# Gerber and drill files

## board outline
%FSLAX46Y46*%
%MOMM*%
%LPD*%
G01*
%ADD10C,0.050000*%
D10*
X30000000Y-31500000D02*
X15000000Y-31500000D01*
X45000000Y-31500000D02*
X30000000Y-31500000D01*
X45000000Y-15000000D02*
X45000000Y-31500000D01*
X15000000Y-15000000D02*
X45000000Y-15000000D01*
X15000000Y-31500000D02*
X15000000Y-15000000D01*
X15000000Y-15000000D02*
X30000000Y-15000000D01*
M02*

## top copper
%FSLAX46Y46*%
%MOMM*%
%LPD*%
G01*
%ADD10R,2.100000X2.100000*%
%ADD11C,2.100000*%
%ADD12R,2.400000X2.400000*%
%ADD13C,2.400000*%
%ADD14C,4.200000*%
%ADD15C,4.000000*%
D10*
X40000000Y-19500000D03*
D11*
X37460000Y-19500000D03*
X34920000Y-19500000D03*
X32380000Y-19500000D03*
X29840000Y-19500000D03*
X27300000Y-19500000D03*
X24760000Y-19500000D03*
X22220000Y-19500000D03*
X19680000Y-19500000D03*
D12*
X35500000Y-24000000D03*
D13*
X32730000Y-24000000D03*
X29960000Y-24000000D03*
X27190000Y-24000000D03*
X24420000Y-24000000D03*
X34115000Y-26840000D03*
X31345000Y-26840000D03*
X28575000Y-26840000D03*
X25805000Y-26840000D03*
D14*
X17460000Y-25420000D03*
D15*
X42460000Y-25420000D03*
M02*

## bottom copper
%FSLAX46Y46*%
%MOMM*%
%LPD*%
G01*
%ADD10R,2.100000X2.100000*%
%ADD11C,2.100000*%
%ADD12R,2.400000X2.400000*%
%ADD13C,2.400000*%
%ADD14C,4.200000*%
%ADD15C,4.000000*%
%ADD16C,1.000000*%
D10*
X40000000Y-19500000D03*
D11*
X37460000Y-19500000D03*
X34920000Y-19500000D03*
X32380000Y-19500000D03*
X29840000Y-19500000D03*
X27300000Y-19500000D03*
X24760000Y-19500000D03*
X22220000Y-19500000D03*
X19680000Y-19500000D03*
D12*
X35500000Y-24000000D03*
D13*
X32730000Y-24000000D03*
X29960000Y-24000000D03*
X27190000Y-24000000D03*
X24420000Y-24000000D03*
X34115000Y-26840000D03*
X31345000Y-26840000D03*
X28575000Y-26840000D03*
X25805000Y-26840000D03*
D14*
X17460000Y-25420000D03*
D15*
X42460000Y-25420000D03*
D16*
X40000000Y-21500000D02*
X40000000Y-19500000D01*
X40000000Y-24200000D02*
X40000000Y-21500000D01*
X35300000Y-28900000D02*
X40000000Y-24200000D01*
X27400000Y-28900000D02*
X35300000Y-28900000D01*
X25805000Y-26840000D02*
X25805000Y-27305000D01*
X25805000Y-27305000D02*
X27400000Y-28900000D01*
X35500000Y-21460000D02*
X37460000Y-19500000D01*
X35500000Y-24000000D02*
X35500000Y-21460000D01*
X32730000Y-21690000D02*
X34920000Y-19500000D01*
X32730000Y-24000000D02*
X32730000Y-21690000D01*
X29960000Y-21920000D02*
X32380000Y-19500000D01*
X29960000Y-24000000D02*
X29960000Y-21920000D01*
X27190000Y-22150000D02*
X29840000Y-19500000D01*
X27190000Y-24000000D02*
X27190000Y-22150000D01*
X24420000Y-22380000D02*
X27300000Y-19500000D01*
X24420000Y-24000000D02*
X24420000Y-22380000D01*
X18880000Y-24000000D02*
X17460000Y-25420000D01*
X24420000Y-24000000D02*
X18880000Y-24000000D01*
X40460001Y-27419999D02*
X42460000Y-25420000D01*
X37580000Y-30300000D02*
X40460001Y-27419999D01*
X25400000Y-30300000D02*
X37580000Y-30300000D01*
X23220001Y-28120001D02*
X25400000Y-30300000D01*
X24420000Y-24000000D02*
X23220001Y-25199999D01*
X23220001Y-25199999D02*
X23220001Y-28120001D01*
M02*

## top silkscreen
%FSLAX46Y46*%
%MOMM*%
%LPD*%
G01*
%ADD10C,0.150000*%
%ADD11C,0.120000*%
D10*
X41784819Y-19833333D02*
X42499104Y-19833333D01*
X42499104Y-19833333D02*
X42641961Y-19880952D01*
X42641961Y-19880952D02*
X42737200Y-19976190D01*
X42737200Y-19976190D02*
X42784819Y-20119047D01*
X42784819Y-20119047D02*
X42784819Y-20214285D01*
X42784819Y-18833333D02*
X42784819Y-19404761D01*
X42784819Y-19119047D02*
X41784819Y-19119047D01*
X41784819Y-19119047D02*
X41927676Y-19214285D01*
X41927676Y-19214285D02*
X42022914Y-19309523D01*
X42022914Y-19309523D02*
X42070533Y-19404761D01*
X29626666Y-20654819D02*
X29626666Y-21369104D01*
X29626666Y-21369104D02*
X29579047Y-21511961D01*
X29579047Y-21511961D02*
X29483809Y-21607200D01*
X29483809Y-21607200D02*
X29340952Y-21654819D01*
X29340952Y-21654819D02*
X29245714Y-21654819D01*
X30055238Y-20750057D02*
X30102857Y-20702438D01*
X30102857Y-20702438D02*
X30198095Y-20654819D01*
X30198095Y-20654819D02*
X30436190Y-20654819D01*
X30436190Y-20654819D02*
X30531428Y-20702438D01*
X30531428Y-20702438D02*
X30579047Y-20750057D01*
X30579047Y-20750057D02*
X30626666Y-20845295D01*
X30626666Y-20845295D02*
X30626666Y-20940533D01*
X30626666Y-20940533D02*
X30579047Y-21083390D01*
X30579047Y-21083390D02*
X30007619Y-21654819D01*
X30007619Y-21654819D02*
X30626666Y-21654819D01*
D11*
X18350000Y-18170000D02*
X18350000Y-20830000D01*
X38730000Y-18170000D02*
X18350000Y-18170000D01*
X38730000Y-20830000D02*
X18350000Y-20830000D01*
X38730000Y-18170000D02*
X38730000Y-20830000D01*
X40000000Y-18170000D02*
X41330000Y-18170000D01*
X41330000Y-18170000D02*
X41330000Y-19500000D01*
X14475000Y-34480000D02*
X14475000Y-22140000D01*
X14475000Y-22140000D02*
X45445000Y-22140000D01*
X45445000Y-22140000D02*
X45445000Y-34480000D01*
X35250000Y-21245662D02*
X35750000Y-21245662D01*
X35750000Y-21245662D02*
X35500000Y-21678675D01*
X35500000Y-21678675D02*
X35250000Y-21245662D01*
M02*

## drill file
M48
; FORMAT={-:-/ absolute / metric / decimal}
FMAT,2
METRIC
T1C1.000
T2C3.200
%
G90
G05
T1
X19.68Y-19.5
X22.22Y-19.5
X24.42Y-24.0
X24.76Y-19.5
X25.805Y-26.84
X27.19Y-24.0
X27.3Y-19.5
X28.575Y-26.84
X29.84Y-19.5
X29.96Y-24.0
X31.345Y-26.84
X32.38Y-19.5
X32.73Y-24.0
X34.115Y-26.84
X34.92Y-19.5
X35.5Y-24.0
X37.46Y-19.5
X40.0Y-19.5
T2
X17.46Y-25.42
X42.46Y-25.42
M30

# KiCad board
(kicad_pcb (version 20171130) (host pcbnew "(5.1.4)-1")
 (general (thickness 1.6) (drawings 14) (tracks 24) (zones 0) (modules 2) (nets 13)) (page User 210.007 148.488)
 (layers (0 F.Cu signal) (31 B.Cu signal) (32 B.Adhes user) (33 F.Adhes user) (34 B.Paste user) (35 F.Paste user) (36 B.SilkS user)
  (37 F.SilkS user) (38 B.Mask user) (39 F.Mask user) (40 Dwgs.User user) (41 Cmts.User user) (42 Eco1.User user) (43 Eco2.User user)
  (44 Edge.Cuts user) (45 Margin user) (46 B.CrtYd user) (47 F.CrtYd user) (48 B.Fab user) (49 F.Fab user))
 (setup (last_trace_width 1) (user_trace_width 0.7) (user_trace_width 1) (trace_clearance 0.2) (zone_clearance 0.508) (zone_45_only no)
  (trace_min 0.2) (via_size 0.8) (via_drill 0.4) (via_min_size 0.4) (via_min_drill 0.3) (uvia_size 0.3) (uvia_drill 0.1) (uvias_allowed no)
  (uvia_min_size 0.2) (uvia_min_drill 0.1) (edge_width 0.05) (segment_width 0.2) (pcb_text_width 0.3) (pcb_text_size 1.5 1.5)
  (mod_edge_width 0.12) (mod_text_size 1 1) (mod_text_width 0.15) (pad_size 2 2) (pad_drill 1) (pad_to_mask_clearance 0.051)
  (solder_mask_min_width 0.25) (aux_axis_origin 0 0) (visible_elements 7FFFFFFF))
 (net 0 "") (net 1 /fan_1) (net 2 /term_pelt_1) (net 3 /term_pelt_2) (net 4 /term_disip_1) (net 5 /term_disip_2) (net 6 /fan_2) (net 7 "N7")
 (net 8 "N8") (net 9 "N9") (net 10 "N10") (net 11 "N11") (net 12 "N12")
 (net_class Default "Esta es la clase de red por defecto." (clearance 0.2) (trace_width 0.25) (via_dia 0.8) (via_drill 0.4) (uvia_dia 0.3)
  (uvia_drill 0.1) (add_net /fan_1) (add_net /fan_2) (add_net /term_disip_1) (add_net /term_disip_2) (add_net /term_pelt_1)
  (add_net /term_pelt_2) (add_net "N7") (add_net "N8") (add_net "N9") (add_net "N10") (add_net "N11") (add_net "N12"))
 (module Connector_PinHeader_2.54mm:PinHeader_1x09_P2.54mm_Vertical (layer F.Cu) (at 40 19.5 270)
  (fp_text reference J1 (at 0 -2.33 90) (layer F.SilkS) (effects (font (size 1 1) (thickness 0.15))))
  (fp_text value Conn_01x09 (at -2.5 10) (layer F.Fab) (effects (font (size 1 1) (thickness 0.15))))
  (fp_line (start -1.33 21.65) (end 1.33 21.65) (layer F.SilkS) (width 0.12))
  (fp_line (start -1.33 1.27) (end -1.33 21.65) (layer F.SilkS) (width 0.12))
  (fp_line (start 1.33 1.27) (end 1.33 21.65) (layer F.SilkS) (width 0.12))
  (fp_line (start -1.33 1.27) (end 1.33 1.27) (layer F.SilkS) (width 0.12))
  (fp_line (start -1.33 0) (end -1.33 -1.33) (layer F.SilkS) (width 0.12))
  (fp_line (start -1.33 -1.33) (end 0 -1.33) (layer F.SilkS) (width 0.12))
  (pad 1 thru_hole rect (at 0 0 270) (size 2.1 2.1) (drill 1) (layers *.Cu *.Mask) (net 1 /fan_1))
  (pad 2 thru_hole circle (at 0 2.54 270) (size 2.1 2.1) (drill 1) (layers *.Cu *.Mask) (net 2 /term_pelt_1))
  (pad 3 thru_hole circle (at 0 5.08 270) (size 2.1 2.1) (drill 1) (layers *.Cu *.Mask) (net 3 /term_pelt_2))
  (pad 4 thru_hole circle (at 0 7.62 270) (size 2.1 2.1) (drill 1) (layers *.Cu *.Mask) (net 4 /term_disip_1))
  (pad 5 thru_hole circle (at 0 10.16 270) (size 2.1 2.1) (drill 1) (layers *.Cu *.Mask) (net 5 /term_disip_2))
  (pad 6 thru_hole circle (at 0 12.7 270) (size 2.1 2.1) (drill 1) (layers *.Cu *.Mask) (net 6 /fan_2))
  (pad 7 thru_hole circle (at 0 15.24 270) (size 2.1 2.1) (drill 1) (layers *.Cu *.Mask) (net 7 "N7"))
  (pad 8 thru_hole circle (at 0 17.78 270) (size 2.1 2.1) (drill 1) (layers *.Cu *.Mask) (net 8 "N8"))
  (pad 9 thru_hole circle (at 0 20.32 270) (size 2.1 2.1) (drill 1) (layers *.Cu *.Mask) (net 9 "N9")))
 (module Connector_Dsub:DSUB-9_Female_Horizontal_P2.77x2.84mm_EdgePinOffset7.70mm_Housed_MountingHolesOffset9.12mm (layer F.Cu) (at 35.5 24)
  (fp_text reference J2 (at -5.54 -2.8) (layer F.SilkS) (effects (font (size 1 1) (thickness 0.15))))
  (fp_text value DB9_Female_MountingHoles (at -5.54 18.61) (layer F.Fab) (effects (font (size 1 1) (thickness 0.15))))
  (fp_line (start -21.025 10.48) (end -21.025 -1.86) (layer F.SilkS) (width 0.12))
  (fp_line (start -21.025 -1.86) (end 9.945 -1.86) (layer F.SilkS) (width 0.12))
  (fp_line (start 9.945 -1.86) (end 9.945 10.48) (layer F.SilkS) (width 0.12))
  (fp_line (start -0.25 -2.754338) (end 0.25 -2.754338) (layer F.SilkS) (width 0.12))
  (fp_line (start 0.25 -2.754338) (end 0 -2.321325) (layer F.SilkS) (width 0.12))
  (fp_line (start 0 -2.321325) (end -0.25 -2.754338) (layer F.SilkS) (width 0.12))
  (pad 1 thru_hole rect (at 0 0) (size 2.4 2.4) (drill 1) (layers *.Cu *.Mask) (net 2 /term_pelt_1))
  (pad 2 thru_hole circle (at -2.77 0) (size 2.4 2.4) (drill 1) (layers *.Cu *.Mask) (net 3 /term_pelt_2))
  (pad 3 thru_hole circle (at -5.54 0) (size 2.4 2.4) (drill 1) (layers *.Cu *.Mask) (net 4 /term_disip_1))
  (pad 4 thru_hole circle (at -8.31 0) (size 2.4 2.4) (drill 1) (layers *.Cu *.Mask) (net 5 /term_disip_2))
  (pad 5 thru_hole circle (at -11.08 0) (size 2.4 2.4) (drill 1) (layers *.Cu *.Mask) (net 6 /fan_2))
  (pad 6 thru_hole circle (at -1.385 2.84) (size 2.4 2.4) (drill 1) (layers *.Cu *.Mask) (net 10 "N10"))
  (pad 7 thru_hole circle (at -4.155 2.84) (size 2.4 2.4) (drill 1) (layers *.Cu *.Mask) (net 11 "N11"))
  (pad 8 thru_hole circle (at -6.925 2.84) (size 2.4 2.4) (drill 1) (layers *.Cu *.Mask) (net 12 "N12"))
  (pad 9 thru_hole circle (at -9.695 2.84) (size 2.4 2.4) (drill 1) (layers *.Cu *.Mask) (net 1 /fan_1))
  (pad 0 thru_hole circle (at -18.04 1.42) (size 4.2 4.2) (drill 3.2) (layers *.Cu *.Mask) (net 6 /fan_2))
  (pad 0 thru_hole circle (at 6.96 1.42) (size 4 4) (drill 3.2) (layers *.Cu *.Mask) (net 6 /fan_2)))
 (gr_line (start 30 31.5) (end 15 31.5) (layer Edge.Cuts) (width 0.05))
 (gr_line (start 45 31.5) (end 30 31.5) (layer Edge.Cuts) (width 0.05))
 (gr_line (start 45 15) (end 45 31.5) (layer Edge.Cuts) (width 0.05))
 (gr_line (start 15 15) (end 45 15) (layer Edge.Cuts) (width 0.05))
 (gr_line (start 15 31.5) (end 15 15) (layer Edge.Cuts) (width 0.05))
 (gr_line (start 15 15) (end 30 15) (layer Edge.Cuts) (width 0.05))
 (segment (start 40 21.5) (end 40 19.5) (width 1) (layer B.Cu) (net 1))
 (segment (start 40 24.2) (end 40 21.5) (width 1) (layer B.Cu) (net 1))
 (segment (start 35.3 28.9) (end 40 24.2) (width 1) (layer B.Cu) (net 1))
 (segment (start 27.4 28.9) (end 35.3 28.9) (width 1) (layer B.Cu) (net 1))
 (segment (start 25.805 26.84) (end 25.805 27.305) (width 1) (layer B.Cu) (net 1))
 (segment (start 25.805 27.305) (end 27.4 28.9) (width 1) (layer B.Cu) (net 1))
 (segment (start 35.5 21.46) (end 37.46 19.5) (width 1) (layer B.Cu) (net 2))
 (segment (start 35.5 24) (end 35.5 21.46) (width 1) (layer B.Cu) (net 2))
 (segment (start 32.73 21.69) (end 34.92 19.5) (width 1) (layer B.Cu) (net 3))
 (segment (start 32.73 24) (end 32.73 21.69) (width 1) (layer B.Cu) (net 3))
 (segment (start 29.96 21.92) (end 32.38 19.5) (width 1) (layer B.Cu) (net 4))
 (segment (start 29.96 24) (end 29.96 21.92) (width 1) (layer B.Cu) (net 4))
 (segment (start 27.19 22.15) (end 29.84 19.5) (width 1) (layer B.Cu) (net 5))
 (segment (start 27.19 24) (end 27.19 22.15) (width 1) (layer B.Cu) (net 5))
 (segment (start 24.42 22.38) (end 27.3 19.5) (width 1) (layer B.Cu) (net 6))
 (segment (start 24.42 24) (end 24.42 22.38) (width 1) (layer B.Cu) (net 6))
 (segment (start 18.88 24) (end 17.46 25.42) (width 1) (layer B.Cu) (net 6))
 (segment (start 24.42 24) (end 18.88 24) (width 1) (layer B.Cu) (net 6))
 (segment (start 40.460001 27.419999) (end 42.46 25.42) (width 1) (layer B.Cu) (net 6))
 (segment (start 37.58 30.3) (end 40.460001 27.419999) (width 1) (layer B.Cu) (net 6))
 (segment (start 25.4 30.3) (end 37.58 30.3) (width 1) (layer B.Cu) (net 6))
 (segment (start 23.220001 28.120001) (end 25.4 30.3) (width 1) (layer B.Cu) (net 6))
 (segment (start 24.42 24) (end 23.220001 25.199999) (width 1) (layer B.Cu) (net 6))
 (segment (start 23.220001 25.199999) (end 23.220001 28.120001) (width 1) (layer B.Cu) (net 6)))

